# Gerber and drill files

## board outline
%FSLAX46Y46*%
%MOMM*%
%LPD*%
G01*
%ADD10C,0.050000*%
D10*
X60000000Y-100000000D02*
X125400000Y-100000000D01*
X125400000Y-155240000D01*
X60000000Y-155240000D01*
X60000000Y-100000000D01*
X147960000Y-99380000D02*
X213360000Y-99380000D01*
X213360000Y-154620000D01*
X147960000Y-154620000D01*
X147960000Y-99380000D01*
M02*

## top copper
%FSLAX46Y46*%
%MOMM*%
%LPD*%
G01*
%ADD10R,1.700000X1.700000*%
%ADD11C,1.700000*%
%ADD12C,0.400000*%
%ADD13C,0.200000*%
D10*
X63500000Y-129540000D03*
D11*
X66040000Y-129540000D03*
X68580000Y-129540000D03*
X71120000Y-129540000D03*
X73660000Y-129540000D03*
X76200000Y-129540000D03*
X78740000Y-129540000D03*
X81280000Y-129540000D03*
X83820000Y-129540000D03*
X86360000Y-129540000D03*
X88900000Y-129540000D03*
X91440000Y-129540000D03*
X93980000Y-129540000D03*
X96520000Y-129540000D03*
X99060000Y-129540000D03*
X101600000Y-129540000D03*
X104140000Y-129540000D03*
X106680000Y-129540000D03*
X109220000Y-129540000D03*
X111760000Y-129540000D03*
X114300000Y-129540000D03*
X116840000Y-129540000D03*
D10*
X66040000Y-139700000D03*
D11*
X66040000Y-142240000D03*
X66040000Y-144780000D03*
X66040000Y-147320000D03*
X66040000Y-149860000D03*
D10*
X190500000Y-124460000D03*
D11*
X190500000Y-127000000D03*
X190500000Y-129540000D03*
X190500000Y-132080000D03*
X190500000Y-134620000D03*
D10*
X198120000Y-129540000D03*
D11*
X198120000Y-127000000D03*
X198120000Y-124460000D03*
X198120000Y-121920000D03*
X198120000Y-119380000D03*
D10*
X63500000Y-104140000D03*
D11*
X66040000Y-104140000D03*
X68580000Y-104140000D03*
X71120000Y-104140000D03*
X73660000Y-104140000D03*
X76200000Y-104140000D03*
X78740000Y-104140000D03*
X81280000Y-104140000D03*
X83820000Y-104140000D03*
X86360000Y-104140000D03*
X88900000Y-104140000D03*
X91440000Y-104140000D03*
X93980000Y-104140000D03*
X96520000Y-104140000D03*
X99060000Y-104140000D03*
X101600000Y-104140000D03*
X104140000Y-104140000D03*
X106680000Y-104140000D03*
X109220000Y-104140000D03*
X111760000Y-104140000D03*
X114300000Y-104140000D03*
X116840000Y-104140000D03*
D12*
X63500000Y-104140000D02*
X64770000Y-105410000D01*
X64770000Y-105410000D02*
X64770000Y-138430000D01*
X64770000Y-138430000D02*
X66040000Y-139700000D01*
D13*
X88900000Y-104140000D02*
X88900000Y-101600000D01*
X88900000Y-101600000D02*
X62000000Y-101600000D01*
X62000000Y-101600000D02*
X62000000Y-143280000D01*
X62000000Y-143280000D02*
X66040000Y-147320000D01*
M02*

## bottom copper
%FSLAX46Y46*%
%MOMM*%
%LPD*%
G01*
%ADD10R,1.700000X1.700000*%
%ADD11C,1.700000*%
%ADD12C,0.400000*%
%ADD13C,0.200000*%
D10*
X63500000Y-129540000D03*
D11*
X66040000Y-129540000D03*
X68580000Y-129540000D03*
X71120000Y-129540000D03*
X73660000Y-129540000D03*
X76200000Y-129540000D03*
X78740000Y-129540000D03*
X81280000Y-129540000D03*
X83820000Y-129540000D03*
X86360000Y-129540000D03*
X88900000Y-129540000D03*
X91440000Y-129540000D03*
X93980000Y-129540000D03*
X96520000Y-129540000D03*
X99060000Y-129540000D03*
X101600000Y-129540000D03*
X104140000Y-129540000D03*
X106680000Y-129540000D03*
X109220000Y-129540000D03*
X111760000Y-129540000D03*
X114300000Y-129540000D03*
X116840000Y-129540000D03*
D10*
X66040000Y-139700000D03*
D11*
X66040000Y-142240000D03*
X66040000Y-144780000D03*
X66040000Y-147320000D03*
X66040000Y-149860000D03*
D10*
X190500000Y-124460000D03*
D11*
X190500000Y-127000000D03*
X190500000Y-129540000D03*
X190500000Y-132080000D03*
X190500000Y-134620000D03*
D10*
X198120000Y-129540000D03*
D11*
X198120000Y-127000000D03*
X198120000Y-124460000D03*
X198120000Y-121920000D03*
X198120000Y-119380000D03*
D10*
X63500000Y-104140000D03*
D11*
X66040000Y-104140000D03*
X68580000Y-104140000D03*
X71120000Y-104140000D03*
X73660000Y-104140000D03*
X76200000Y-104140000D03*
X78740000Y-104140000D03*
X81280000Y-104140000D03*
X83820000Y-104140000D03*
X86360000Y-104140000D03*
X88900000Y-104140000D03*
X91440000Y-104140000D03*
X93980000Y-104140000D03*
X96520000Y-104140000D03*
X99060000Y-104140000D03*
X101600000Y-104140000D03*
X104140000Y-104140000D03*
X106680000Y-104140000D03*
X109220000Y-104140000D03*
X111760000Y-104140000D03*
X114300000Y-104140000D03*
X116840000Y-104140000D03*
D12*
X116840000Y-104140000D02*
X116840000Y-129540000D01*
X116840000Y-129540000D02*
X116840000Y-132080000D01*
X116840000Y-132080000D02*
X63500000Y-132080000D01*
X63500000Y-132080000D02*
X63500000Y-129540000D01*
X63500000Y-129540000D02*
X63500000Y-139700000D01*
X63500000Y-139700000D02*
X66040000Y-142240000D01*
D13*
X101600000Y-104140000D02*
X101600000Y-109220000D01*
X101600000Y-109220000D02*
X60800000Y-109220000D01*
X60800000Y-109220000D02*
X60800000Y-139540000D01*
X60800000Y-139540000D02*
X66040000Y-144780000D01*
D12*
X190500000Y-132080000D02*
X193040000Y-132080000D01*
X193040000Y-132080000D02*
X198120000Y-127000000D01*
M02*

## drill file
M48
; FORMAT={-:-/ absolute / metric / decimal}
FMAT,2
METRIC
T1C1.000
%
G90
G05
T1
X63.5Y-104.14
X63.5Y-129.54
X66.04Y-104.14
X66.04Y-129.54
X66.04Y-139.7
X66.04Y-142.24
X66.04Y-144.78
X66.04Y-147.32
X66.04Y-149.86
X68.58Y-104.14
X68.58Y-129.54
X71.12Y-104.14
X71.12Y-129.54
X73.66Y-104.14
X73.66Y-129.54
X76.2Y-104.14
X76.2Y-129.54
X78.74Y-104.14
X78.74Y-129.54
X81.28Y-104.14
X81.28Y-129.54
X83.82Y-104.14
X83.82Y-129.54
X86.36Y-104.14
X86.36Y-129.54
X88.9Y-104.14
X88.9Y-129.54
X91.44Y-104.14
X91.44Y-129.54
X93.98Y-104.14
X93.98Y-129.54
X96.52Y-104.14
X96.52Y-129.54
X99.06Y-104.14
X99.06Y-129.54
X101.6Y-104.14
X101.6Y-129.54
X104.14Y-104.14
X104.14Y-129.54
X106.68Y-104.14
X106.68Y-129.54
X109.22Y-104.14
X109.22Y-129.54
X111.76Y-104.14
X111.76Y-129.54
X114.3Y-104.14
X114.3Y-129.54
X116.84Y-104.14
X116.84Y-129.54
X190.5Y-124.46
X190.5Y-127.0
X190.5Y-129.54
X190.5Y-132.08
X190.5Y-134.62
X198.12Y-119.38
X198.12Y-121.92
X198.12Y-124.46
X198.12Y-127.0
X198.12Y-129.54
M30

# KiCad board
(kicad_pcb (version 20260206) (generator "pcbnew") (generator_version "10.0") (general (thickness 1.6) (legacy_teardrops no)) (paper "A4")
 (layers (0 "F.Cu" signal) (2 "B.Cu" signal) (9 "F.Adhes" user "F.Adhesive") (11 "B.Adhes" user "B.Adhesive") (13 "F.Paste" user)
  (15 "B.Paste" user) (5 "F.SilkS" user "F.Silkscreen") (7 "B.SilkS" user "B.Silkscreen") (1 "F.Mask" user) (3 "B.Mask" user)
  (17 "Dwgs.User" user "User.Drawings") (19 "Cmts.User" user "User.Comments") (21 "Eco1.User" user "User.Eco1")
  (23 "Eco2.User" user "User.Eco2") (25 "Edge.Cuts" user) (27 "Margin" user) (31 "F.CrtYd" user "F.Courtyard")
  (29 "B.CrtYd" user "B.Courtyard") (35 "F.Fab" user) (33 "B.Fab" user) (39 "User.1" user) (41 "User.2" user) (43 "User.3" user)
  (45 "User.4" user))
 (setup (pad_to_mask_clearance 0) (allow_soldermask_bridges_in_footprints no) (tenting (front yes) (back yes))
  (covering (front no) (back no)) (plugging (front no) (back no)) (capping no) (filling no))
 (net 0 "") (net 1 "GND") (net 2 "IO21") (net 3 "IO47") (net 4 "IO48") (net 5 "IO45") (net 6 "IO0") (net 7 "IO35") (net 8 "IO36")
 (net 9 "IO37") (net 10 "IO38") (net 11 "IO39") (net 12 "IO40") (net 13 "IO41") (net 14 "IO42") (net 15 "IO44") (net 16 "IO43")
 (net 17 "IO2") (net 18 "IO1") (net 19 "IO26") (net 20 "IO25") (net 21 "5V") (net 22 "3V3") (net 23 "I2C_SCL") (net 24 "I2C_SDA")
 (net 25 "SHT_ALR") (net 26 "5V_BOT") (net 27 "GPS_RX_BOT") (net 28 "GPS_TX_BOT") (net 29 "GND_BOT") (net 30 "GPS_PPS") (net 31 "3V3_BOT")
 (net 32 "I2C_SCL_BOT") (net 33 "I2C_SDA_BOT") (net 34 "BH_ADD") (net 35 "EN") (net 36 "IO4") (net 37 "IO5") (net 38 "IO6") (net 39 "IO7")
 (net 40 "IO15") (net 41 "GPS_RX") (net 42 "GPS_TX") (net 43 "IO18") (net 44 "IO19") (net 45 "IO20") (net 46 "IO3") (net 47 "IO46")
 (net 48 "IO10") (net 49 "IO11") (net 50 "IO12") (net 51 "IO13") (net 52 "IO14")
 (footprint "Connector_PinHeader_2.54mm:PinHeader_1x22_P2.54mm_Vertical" (layer "F.Cu") (at 63.5 129.54 90)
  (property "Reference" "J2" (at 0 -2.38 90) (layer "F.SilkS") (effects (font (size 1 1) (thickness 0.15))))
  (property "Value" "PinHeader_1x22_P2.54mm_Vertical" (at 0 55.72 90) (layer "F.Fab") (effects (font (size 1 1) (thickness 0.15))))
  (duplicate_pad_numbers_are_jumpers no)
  (pad "1" thru_hole rect (at 0 0 90) (size 1.7 1.7) (drill 1) (layers "*.Cu" "*.Mask") (remove_unused_layers no) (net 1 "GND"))
  (pad "2" thru_hole circle (at 0 2.54 90) (size 1.7 1.7) (drill 1) (layers "*.Cu" "*.Mask") (remove_unused_layers no) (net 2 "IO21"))
  (pad "3" thru_hole circle (at 0 5.08 90) (size 1.7 1.7) (drill 1) (layers "*.Cu" "*.Mask") (remove_unused_layers no) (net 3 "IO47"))
  (pad "4" thru_hole circle (at 0 7.62 90) (size 1.7 1.7) (drill 1) (layers "*.Cu" "*.Mask") (remove_unused_layers no) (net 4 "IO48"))
  (pad "5" thru_hole circle (at 0 10.16 90) (size 1.7 1.7) (drill 1) (layers "*.Cu" "*.Mask") (remove_unused_layers no) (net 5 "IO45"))
  (pad "6" thru_hole circle (at 0 12.7 90) (size 1.7 1.7) (drill 1) (layers "*.Cu" "*.Mask") (remove_unused_layers no) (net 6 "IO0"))
  (pad "7" thru_hole circle (at 0 15.24 90) (size 1.7 1.7) (drill 1) (layers "*.Cu" "*.Mask") (remove_unused_layers no) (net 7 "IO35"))
  (pad "8" thru_hole circle (at 0 17.78 90) (size 1.7 1.7) (drill 1) (layers "*.Cu" "*.Mask") (remove_unused_layers no) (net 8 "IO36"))
  (pad "9" thru_hole circle (at 0 20.32 90) (size 1.7 1.7) (drill 1) (layers "*.Cu" "*.Mask") (remove_unused_layers no) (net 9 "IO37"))
  (pad "10" thru_hole circle (at 0 22.86 90) (size 1.7 1.7) (drill 1) (layers "*.Cu" "*.Mask") (remove_unused_layers no) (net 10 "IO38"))
  (pad "11" thru_hole circle (at 0 25.4 90) (size 1.7 1.7) (drill 1) (layers "*.Cu" "*.Mask") (remove_unused_layers no) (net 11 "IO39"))
  (pad "12" thru_hole circle (at 0 27.94 90) (size 1.7 1.7) (drill 1) (layers "*.Cu" "*.Mask") (remove_unused_layers no) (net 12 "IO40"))
  (pad "13" thru_hole circle (at 0 30.48 90) (size 1.7 1.7) (drill 1) (layers "*.Cu" "*.Mask") (remove_unused_layers no) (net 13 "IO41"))
  (pad "14" thru_hole circle (at 0 33.02 90) (size 1.7 1.7) (drill 1) (layers "*.Cu" "*.Mask") (remove_unused_layers no) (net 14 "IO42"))
  (pad "15" thru_hole circle (at 0 35.56 90) (size 1.7 1.7) (drill 1) (layers "*.Cu" "*.Mask") (remove_unused_layers no) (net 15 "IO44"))
  (pad "16" thru_hole circle (at 0 38.1 90) (size 1.7 1.7) (drill 1) (layers "*.Cu" "*.Mask") (remove_unused_layers no) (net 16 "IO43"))
  (pad "17" thru_hole circle (at 0 40.64 90) (size 1.7 1.7) (drill 1) (layers "*.Cu" "*.Mask") (remove_unused_layers no) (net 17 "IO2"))
  (pad "18" thru_hole circle (at 0 43.18 90) (size 1.7 1.7) (drill 1) (layers "*.Cu" "*.Mask") (remove_unused_layers no) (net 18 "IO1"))
  (pad "19" thru_hole circle (at 0 45.72 90) (size 1.7 1.7) (drill 1) (layers "*.Cu" "*.Mask") (remove_unused_layers no) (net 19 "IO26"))
  (pad "20" thru_hole circle (at 0 48.26 90) (size 1.7 1.7) (drill 1) (layers "*.Cu" "*.Mask") (remove_unused_layers no) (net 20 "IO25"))
  (pad "21" thru_hole circle (at 0 50.8 90) (size 1.7 1.7) (drill 1) (layers "*.Cu" "*.Mask") (remove_unused_layers no) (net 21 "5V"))
  (pad "22" thru_hole circle (at 0 53.34 90) (size 1.7 1.7) (drill 1) (layers "*.Cu" "*.Mask") (remove_unused_layers no) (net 1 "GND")))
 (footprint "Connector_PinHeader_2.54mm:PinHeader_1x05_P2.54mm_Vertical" (layer "F.Cu") (at 66.04 139.7)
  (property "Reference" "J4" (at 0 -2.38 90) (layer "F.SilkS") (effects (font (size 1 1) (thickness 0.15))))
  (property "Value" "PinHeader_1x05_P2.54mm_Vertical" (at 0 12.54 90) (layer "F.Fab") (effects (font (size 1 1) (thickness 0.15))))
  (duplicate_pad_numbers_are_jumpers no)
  (pad "1" thru_hole rect (at 0 0 90) (size 1.7 1.7) (drill 1) (layers "*.Cu" "*.Mask") (remove_unused_layers no) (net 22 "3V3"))
  (pad "2" thru_hole circle (at 0 2.54 90) (size 1.7 1.7) (drill 1) (layers "*.Cu" "*.Mask") (remove_unused_layers no) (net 1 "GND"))
  (pad "3" thru_hole circle (at 0 5.08 90) (size 1.7 1.7) (drill 1) (layers "*.Cu" "*.Mask") (remove_unused_layers no) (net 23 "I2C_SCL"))
  (pad "4" thru_hole circle (at 0 7.62 90) (size 1.7 1.7) (drill 1) (layers "*.Cu" "*.Mask") (remove_unused_layers no) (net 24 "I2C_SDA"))
  (pad "5" thru_hole circle (at 0 10.16 90) (size 1.7 1.7) (drill 1) (layers "*.Cu" "*.Mask") (remove_unused_layers no) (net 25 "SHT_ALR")))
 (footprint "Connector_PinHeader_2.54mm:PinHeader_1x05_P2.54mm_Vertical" (layer "F.Cu") (at 190.5 124.46)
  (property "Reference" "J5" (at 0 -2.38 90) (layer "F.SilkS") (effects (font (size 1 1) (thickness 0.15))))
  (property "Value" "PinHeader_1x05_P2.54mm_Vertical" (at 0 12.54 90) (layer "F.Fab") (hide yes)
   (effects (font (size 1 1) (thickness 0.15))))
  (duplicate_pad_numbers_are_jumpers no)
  (pad "1" thru_hole rect (at 0 0 90) (size 1.7 1.7) (drill 1) (layers "*.Cu" "*.Mask") (remove_unused_layers no) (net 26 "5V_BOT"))
  (pad "2" thru_hole circle (at 0 2.54 90) (size 1.7 1.7) (drill 1) (layers "*.Cu" "*.Mask") (remove_unused_layers no) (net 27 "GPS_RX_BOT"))
  (pad "3" thru_hole circle (at 0 5.08 90) (size 1.7 1.7) (drill 1) (layers "*.Cu" "*.Mask") (remove_unused_layers no) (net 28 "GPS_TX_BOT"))
  (pad "4" thru_hole circle (at 0 7.62 90) (size 1.7 1.7) (drill 1) (layers "*.Cu" "*.Mask") (remove_unused_layers no) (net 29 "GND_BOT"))
  (pad "5" thru_hole circle (at 0 10.16 90) (size 1.7 1.7) (drill 1) (layers "*.Cu" "*.Mask") (remove_unused_layers no) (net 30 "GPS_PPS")))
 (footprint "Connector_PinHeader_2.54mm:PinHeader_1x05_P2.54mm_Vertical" (layer "F.Cu") (at 198.12 129.54 180)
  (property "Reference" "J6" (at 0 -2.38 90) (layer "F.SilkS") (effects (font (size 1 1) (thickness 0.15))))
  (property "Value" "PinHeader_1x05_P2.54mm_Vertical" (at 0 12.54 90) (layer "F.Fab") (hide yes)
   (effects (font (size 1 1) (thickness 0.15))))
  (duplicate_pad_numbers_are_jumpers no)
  (pad "1" thru_hole rect (at 0 0 270) (size 1.7 1.7) (drill 1) (layers "*.Cu" "*.Mask") (remove_unused_layers no) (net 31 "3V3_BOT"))
  (pad "2" thru_hole circle (at 0 2.54 270) (size 1.7 1.7) (drill 1) (layers "*.Cu" "*.Mask") (remove_unused_layers no) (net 29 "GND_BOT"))
  (pad "3" thru_hole circle (at 0 5.08 270) (size 1.7 1.7) (drill 1) (layers "*.Cu" "*.Mask") (remove_unused_layers no)
   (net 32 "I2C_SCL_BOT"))
  (pad "4" thru_hole circle (at 0 7.62 270) (size 1.7 1.7) (drill 1) (layers "*.Cu" "*.Mask") (remove_unused_layers no)
   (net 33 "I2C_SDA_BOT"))
  (pad "5" thru_hole circle (at 0 10.16 270) (size 1.7 1.7) (drill 1) (layers "*.Cu" "*.Mask") (remove_unused_layers no) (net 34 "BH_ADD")))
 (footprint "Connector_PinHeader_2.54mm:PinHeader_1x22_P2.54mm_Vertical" (layer "F.Cu") (at 63.5 104.14 90)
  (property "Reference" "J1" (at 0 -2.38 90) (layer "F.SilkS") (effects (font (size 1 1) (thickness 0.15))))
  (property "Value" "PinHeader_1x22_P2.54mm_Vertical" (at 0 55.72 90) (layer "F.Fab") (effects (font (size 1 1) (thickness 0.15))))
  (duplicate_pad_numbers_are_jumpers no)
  (pad "1" thru_hole rect (at 0 0 90) (size 1.7 1.7) (drill 1) (layers "*.Cu" "*.Mask") (remove_unused_layers no) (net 22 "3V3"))
  (pad "2" thru_hole circle (at 0 2.54 90) (size 1.7 1.7) (drill 1) (layers "*.Cu" "*.Mask") (remove_unused_layers no) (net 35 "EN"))
  (pad "3" thru_hole circle (at 0 5.08 90) (size 1.7 1.7) (drill 1) (layers "*.Cu" "*.Mask") (remove_unused_layers no) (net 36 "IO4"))
  (pad "4" thru_hole circle (at 0 7.62 90) (size 1.7 1.7) (drill 1) (layers "*.Cu" "*.Mask") (remove_unused_layers no) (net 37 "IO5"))
  (pad "5" thru_hole circle (at 0 10.16 90) (size 1.7 1.7) (drill 1) (layers "*.Cu" "*.Mask") (remove_unused_layers no) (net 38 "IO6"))
  (pad "6" thru_hole circle (at 0 12.7 90) (size 1.7 1.7) (drill 1) (layers "*.Cu" "*.Mask") (remove_unused_layers no) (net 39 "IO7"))
  (pad "7" thru_hole circle (at 0 15.24 90) (size 1.7 1.7) (drill 1) (layers "*.Cu" "*.Mask") (remove_unused_layers no) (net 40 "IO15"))
  (pad "8" thru_hole circle (at 0 17.78 90) (size 1.7 1.7) (drill 1) (layers "*.Cu" "*.Mask") (remove_unused_layers no) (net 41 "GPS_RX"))
  (pad "9" thru_hole circle (at 0 20.32 90) (size 1.7 1.7) (drill 1) (layers "*.Cu" "*.Mask") (remove_unused_layers no) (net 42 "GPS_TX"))
  (pad "10" thru_hole circle (at 0 22.86 90) (size 1.7 1.7) (drill 1) (layers "*.Cu" "*.Mask") (remove_unused_layers no) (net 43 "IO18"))
  (pad "11" thru_hole circle (at 0 25.4 90) (size 1.7 1.7) (drill 1) (layers "*.Cu" "*.Mask") (remove_unused_layers no) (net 24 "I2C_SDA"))
  (pad "12" thru_hole circle (at 0 27.94 90) (size 1.7 1.7) (drill 1) (layers "*.Cu" "*.Mask") (remove_unused_layers no) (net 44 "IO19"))
  (pad "13" thru_hole circle (at 0 30.48 90) (size 1.7 1.7) (drill 1) (layers "*.Cu" "*.Mask") (remove_unused_layers no) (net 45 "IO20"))
  (pad "14" thru_hole circle (at 0 33.02 90) (size 1.7 1.7) (drill 1) (layers "*.Cu" "*.Mask") (remove_unused_layers no) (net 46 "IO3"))
  (pad "15" thru_hole circle (at 0 35.56 90) (size 1.7 1.7) (drill 1) (layers "*.Cu" "*.Mask") (remove_unused_layers no) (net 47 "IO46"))
  (pad "16" thru_hole circle (at 0 38.1 90) (size 1.7 1.7) (drill 1) (layers "*.Cu" "*.Mask") (remove_unused_layers no) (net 23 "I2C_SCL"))
  (pad "17" thru_hole circle (at 0 40.64 90) (size 1.7 1.7) (drill 1) (layers "*.Cu" "*.Mask") (remove_unused_layers no) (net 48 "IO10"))
  (pad "18" thru_hole circle (at 0 43.18 90) (size 1.7 1.7) (drill 1) (layers "*.Cu" "*.Mask") (remove_unused_layers no) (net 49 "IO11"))
  (pad "19" thru_hole circle (at 0 45.72 90) (size 1.7 1.7) (drill 1) (layers "*.Cu" "*.Mask") (remove_unused_layers no) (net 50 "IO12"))
  (pad "20" thru_hole circle (at 0 48.26 90) (size 1.7 1.7) (drill 1) (layers "*.Cu" "*.Mask") (remove_unused_layers no) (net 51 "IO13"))
  (pad "21" thru_hole circle (at 0 50.8 90) (size 1.7 1.7) (drill 1) (layers "*.Cu" "*.Mask") (remove_unused_layers no) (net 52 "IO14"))
  (pad "22" thru_hole circle (at 0 53.34 90) (size 1.7 1.7) (drill 1) (layers "*.Cu" "*.Mask") (remove_unused_layers no) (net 1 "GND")))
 (gr_rect (start 60 100) (end 125.4 155.24) (stroke (width 0.05) (type solid)) (fill no) (layer "Edge.Cuts"))
 (gr_rect (start 147.96 99.38) (end 213.36 154.62) (stroke (width 0.05) (type solid)) (fill no) (layer "Edge.Cuts"))
 (segment (start 63.5 104.14) (end 64.77 105.41) (width 0.4) (layer "F.Cu") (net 22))
 (segment (start 64.77 105.41) (end 64.77 138.43) (width 0.4) (layer "F.Cu") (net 22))
 (segment (start 64.77 138.43) (end 66.04 139.7) (width 0.4) (layer "F.Cu") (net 22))
 (segment (start 116.84 104.14) (end 116.84 129.54) (width 0.4) (layer "B.Cu") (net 1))
 (segment (start 116.84 129.54) (end 116.84 132.08) (width 0.4) (layer "B.Cu") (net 1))
 (segment (start 116.84 132.08) (end 63.5 132.08) (width 0.4) (layer "B.Cu") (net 1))
 (segment (start 63.5 132.08) (end 63.5 129.54) (width 0.4) (layer "B.Cu") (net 1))
 (segment (start 63.5 129.54) (end 63.5 139.7) (width 0.4) (layer "B.Cu") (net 1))
 (segment (start 63.5 139.7) (end 66.04 142.24) (width 0.4) (layer "B.Cu") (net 1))
 (segment (start 88.9 104.14) (end 88.9 101.6) (width 0.2) (layer "F.Cu") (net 24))
 (segment (start 88.9 101.6) (end 62.0 101.6) (width 0.2) (layer "F.Cu") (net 24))
 (segment (start 62.0 101.6) (end 62.0 143.28) (width 0.2) (layer "F.Cu") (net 24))
 (segment (start 62.0 143.28) (end 66.04 147.32) (width 0.2) (layer "F.Cu") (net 24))
 (segment (start 101.6 104.14) (end 101.6 109.22) (width 0.2) (layer "B.Cu") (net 23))
 (segment (start 101.6 109.22) (end 60.8 109.22) (width 0.2) (layer "B.Cu") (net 23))
 (segment (start 60.8 109.22) (end 60.8 139.54) (width 0.2) (layer "B.Cu") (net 23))
 (segment (start 60.8 139.54) (end 66.04 144.78) (width 0.2) (layer "B.Cu") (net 23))
 (segment (start 190.5 132.08) (end 193.04 132.08) (width 0.4) (layer "B.Cu") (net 29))
 (segment (start 193.04 132.08) (end 198.12 127.0) (width 0.4) (layer "B.Cu") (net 29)))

